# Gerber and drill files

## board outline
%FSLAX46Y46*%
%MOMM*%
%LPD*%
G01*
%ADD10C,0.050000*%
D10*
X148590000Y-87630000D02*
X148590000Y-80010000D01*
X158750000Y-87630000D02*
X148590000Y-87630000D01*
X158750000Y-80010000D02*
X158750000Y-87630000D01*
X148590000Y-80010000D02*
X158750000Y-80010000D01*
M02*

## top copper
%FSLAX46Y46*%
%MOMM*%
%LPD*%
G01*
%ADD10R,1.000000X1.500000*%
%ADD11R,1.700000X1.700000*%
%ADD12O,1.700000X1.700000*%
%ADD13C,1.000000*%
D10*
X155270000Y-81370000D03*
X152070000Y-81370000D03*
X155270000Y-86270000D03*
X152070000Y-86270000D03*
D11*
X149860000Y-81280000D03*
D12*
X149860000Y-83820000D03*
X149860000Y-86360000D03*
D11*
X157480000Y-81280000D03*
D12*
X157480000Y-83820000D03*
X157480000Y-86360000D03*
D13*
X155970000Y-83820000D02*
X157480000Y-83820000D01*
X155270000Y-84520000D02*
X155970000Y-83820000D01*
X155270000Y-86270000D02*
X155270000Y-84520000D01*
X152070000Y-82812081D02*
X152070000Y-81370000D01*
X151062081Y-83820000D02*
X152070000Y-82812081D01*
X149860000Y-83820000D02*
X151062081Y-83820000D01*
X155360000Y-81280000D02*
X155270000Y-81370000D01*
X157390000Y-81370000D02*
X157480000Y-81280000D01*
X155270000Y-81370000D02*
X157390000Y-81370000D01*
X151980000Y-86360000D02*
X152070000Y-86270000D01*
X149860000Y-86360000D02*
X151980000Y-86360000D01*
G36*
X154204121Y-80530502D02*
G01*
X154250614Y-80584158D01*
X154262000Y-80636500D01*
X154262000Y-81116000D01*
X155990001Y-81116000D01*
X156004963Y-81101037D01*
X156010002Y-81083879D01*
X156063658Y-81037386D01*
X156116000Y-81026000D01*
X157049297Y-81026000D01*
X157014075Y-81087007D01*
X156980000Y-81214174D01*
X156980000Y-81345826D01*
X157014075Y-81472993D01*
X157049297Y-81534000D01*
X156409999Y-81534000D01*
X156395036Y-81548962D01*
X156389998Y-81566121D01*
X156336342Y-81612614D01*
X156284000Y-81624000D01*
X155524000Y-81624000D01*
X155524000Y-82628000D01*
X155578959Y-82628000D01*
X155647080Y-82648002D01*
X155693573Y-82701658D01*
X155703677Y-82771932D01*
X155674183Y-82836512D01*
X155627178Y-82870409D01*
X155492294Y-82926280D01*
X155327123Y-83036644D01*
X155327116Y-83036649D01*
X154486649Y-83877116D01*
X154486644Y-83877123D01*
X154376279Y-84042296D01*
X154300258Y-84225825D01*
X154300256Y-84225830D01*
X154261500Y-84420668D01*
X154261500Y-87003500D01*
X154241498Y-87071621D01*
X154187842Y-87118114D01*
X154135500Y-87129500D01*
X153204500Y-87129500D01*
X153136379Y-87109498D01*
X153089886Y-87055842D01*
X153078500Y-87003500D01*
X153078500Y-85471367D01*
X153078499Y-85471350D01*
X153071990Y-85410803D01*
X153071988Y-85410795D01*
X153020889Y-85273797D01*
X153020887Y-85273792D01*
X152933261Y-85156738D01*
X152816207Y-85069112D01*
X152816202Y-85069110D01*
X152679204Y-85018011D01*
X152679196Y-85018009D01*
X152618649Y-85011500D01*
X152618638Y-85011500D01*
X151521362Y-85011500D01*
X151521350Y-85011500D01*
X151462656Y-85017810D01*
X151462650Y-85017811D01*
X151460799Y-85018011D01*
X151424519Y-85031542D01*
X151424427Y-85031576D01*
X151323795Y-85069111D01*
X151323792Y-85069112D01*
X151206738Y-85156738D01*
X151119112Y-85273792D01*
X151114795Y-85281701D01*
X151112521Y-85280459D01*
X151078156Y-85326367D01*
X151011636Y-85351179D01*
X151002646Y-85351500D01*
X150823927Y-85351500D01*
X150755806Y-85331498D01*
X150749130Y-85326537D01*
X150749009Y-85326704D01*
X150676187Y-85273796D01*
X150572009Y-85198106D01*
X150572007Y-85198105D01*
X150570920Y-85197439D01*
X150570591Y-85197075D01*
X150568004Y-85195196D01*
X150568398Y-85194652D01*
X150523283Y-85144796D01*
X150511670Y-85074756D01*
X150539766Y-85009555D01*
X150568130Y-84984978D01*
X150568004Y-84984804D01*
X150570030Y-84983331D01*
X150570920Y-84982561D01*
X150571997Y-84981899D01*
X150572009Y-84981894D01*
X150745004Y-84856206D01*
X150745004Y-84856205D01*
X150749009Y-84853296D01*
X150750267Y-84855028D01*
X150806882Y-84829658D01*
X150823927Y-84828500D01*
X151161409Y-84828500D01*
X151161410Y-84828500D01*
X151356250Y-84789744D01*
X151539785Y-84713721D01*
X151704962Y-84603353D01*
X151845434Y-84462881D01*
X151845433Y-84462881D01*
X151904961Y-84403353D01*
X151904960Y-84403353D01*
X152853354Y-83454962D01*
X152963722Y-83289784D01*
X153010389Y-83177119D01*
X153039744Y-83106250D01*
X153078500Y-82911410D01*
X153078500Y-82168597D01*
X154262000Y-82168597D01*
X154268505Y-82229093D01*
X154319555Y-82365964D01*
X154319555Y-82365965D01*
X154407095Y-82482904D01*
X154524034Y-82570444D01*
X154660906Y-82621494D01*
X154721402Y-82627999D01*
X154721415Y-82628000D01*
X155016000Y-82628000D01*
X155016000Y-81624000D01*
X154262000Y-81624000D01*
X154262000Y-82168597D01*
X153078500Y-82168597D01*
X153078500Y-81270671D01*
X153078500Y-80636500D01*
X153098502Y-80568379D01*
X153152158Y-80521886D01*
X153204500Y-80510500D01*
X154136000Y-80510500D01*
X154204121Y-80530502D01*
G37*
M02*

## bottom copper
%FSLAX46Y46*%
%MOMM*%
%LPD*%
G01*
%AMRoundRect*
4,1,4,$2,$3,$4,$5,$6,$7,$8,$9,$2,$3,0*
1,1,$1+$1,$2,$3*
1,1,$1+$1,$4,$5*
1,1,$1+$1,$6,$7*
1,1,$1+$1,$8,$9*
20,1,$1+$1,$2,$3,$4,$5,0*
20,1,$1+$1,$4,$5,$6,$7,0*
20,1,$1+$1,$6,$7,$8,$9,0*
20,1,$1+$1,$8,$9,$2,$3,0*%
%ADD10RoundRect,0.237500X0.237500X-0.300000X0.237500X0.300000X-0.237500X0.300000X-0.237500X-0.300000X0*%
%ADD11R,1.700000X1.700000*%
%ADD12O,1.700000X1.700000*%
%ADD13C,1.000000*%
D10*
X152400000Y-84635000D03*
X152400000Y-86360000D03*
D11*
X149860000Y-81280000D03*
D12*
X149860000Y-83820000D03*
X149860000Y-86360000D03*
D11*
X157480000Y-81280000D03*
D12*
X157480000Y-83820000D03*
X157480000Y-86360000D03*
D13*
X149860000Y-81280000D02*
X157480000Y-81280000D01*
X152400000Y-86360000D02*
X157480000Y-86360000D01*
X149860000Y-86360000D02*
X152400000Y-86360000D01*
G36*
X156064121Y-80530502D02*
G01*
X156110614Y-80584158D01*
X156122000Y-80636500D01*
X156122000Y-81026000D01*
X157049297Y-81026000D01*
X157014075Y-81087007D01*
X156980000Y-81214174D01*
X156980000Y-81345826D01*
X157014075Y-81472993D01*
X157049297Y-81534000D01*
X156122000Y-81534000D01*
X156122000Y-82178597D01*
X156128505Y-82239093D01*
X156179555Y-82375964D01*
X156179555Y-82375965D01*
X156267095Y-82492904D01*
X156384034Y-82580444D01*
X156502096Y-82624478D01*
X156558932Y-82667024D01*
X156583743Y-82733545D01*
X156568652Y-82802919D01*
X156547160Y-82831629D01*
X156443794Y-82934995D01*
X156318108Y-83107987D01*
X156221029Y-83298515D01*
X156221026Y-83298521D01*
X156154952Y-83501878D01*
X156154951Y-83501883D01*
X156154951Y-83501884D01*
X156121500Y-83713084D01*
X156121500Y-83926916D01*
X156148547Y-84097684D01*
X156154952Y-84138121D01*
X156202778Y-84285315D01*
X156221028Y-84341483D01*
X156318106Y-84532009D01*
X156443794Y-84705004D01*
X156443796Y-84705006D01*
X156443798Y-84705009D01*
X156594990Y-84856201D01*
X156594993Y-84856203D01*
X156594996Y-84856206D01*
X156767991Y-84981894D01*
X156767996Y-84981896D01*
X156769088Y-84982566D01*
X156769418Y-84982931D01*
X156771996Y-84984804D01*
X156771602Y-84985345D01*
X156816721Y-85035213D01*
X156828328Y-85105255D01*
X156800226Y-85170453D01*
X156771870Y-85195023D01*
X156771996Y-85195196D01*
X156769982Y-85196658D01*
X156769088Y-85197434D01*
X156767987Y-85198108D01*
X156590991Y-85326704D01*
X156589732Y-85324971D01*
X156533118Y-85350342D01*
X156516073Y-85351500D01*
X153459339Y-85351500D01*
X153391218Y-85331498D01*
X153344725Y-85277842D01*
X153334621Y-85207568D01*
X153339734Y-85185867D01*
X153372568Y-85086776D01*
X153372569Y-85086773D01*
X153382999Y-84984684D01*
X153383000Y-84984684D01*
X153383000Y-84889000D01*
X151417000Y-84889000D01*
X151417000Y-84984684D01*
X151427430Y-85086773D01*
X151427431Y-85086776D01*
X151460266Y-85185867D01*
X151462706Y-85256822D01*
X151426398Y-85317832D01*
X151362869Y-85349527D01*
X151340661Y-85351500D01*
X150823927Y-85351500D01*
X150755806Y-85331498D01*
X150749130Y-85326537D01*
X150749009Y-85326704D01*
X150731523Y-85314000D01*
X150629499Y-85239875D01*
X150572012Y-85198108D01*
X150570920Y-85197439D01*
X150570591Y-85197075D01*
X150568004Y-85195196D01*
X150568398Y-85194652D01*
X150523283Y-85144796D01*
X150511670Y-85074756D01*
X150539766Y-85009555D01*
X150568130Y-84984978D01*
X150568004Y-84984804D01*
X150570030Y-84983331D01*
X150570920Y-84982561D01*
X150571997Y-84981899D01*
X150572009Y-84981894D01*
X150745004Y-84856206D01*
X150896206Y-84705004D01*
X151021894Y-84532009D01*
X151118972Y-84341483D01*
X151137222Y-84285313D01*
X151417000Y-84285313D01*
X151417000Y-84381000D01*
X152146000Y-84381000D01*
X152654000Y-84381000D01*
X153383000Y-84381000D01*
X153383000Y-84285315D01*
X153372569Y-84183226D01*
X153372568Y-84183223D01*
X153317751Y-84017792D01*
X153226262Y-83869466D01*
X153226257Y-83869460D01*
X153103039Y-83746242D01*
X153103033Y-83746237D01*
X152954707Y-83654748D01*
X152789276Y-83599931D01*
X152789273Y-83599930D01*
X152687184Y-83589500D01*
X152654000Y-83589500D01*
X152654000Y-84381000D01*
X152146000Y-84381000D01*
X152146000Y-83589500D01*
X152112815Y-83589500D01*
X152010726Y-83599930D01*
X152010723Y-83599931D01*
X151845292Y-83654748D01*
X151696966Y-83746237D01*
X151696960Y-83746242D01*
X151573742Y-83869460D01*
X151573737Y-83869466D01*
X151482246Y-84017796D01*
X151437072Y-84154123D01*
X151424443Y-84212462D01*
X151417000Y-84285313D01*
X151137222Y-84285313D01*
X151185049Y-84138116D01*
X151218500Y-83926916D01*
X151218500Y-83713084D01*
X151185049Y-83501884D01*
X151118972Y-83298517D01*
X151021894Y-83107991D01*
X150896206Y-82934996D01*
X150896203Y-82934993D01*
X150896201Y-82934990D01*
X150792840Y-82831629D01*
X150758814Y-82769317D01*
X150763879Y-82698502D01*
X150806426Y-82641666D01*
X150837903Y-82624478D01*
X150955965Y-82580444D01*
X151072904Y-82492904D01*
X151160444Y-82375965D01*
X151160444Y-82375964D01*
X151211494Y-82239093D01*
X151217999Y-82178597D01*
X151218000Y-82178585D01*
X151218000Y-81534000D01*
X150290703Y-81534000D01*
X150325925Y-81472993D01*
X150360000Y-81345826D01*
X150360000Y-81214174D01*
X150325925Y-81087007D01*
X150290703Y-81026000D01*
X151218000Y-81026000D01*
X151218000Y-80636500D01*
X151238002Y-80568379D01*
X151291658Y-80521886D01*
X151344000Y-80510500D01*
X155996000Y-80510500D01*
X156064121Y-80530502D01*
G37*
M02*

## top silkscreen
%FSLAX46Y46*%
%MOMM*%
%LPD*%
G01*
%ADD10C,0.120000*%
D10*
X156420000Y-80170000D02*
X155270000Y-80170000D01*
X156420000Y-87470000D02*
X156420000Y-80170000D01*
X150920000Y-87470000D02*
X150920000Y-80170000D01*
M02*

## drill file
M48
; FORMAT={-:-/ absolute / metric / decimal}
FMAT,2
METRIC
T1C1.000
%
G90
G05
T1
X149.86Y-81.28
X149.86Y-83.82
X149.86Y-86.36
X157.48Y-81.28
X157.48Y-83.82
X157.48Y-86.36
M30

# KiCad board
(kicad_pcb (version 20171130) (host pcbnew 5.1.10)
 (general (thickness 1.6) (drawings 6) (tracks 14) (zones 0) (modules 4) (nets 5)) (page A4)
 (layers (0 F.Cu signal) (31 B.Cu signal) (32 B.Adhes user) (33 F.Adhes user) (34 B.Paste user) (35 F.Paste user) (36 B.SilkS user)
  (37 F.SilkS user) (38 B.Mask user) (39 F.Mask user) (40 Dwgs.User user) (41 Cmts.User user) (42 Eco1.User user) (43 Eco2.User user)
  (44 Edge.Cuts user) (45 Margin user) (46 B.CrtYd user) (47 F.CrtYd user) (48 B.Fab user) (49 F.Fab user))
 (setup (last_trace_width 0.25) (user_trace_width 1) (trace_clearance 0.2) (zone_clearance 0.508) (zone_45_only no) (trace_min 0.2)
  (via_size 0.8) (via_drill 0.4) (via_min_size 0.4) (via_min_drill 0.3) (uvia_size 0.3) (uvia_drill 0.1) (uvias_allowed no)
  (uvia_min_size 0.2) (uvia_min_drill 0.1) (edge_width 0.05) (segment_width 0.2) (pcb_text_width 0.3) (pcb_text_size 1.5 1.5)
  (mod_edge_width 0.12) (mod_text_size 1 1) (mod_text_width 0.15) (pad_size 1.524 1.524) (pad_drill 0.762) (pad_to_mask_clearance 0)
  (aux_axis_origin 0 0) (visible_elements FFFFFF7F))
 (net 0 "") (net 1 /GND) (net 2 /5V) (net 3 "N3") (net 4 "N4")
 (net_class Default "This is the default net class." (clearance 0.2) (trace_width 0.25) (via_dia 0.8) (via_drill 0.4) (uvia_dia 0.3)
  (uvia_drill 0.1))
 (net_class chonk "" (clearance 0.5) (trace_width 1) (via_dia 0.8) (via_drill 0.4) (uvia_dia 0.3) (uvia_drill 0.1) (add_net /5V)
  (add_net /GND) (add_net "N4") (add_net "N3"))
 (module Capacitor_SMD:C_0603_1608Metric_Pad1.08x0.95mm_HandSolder (layer B.Cu) (at 152.4 85.4975 90)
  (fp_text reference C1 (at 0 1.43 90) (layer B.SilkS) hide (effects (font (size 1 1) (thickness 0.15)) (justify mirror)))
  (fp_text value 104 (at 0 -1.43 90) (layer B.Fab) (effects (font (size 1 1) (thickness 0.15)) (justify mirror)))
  (pad 2 smd roundrect (at 0.8625 0 90) (size 1.075 0.95) (layers B.Cu B.Paste B.Mask) (roundrect_rratio 0.25) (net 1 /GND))
  (pad 1 smd roundrect (at -0.8625 0 90) (size 1.075 0.95) (layers B.Cu B.Paste B.Mask) (roundrect_rratio 0.25) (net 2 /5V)))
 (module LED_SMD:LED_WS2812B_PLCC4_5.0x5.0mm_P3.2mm (layer F.Cu) (at 153.67 83.82 90)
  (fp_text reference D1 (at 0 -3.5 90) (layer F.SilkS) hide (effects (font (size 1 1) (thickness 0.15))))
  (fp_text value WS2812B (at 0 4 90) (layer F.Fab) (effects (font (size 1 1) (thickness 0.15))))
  (fp_line (start 3.65 2.75) (end 3.65 1.6) (layer F.SilkS) (width 0.12))
  (fp_line (start -3.65 2.75) (end 3.65 2.75) (layer F.SilkS) (width 0.12))
  (fp_line (start -3.65 -2.75) (end 3.65 -2.75) (layer F.SilkS) (width 0.12))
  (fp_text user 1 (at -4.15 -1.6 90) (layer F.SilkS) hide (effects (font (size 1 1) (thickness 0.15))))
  (pad 3 smd rect (at 2.45 1.6 90) (size 1.5 1) (layers F.Cu F.Paste F.Mask) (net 1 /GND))
  (pad 4 smd rect (at 2.45 -1.6 90) (size 1.5 1) (layers F.Cu F.Paste F.Mask) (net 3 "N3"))
  (pad 2 smd rect (at -2.45 1.6 90) (size 1.5 1) (layers F.Cu F.Paste F.Mask) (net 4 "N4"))
  (pad 1 smd rect (at -2.45 -1.6 90) (size 1.5 1) (layers F.Cu F.Paste F.Mask) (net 2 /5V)))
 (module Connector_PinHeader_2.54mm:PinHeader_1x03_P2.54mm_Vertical (layer B.Cu) (at 149.86 81.28 180)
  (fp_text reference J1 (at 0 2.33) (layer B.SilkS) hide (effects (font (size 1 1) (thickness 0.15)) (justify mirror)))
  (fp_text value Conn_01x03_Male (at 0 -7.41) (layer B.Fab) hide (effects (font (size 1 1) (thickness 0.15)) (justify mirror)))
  (pad 1 thru_hole rect (at 0 0 180) (size 1.7 1.7) (drill 1) (layers *.Cu *.Mask) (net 1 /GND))
  (pad 2 thru_hole oval (at 0 -2.54 180) (size 1.7 1.7) (drill 1) (layers *.Cu *.Mask) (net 3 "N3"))
  (pad 3 thru_hole oval (at 0 -5.08 180) (size 1.7 1.7) (drill 1) (layers *.Cu *.Mask) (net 2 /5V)))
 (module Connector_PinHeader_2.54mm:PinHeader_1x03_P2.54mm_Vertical (layer B.Cu) (at 157.48 81.28 180)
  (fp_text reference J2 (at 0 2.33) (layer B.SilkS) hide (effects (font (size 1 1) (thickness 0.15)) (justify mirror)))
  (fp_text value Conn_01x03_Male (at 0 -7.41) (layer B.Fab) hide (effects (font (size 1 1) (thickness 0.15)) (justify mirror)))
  (pad 1 thru_hole rect (at 0 0 180) (size 1.7 1.7) (drill 1) (layers *.Cu *.Mask) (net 1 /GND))
  (pad 2 thru_hole oval (at 0 -2.54 180) (size 1.7 1.7) (drill 1) (layers *.Cu *.Mask) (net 4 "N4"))
  (pad 3 thru_hole oval (at 0 -5.08 180) (size 1.7 1.7) (drill 1) (layers *.Cu *.Mask) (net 2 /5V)))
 (gr_line (start 148.59 87.63) (end 148.59 80.01) (layer Edge.Cuts) (width 0.05))
 (gr_line (start 158.75 87.63) (end 148.59 87.63) (layer Edge.Cuts) (width 0.05))
 (gr_line (start 158.75 80.01) (end 158.75 87.63) (layer Edge.Cuts) (width 0.05))
 (gr_line (start 148.59 80.01) (end 158.75 80.01) (layer Edge.Cuts) (width 0.05))
 (segment (start 155.97 83.82) (end 157.48 83.82) (width 1) (layer F.Cu) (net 4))
 (segment (start 155.27 84.52) (end 155.97 83.82) (width 1) (layer F.Cu) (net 4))
 (segment (start 155.27 86.27) (end 155.27 84.52) (width 1) (layer F.Cu) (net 4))
 (segment (start 152.07 82.812081) (end 152.07 81.37) (width 1) (layer F.Cu) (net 3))
 (segment (start 151.062081 83.82) (end 152.07 82.812081) (width 1) (layer F.Cu) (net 3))
 (segment (start 149.86 83.82) (end 151.062081 83.82) (width 1) (layer F.Cu) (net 3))
 (segment (start 155.36 81.28) (end 155.27 81.37) (width 1) (layer F.Cu) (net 1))
 (segment (start 157.39 81.37) (end 157.48 81.28) (width 1) (layer F.Cu) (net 1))
 (segment (start 155.27 81.37) (end 157.39 81.37) (width 1) (layer F.Cu) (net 1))
 (segment (start 149.86 81.28) (end 157.48 81.28) (width 1) (layer B.Cu) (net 1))
 (segment (start 151.98 86.36) (end 152.07 86.27) (width 1) (layer F.Cu) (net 2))
 (segment (start 149.86 86.36) (end 151.98 86.36) (width 1) (layer F.Cu) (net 2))
 (segment (start 152.4 86.36) (end 157.48 86.36) (width 1) (layer B.Cu) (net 2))
 (segment (start 149.86 86.36) (end 152.4 86.36) (width 1) (layer B.Cu) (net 2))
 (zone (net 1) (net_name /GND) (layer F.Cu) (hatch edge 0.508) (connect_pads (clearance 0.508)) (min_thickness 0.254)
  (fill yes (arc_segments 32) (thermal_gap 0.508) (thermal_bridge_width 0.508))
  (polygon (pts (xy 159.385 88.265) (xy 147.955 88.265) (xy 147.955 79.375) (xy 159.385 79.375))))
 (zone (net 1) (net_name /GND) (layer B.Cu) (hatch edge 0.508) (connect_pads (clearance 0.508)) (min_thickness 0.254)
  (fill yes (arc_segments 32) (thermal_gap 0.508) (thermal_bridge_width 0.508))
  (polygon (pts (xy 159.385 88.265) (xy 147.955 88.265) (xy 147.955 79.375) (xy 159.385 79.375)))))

